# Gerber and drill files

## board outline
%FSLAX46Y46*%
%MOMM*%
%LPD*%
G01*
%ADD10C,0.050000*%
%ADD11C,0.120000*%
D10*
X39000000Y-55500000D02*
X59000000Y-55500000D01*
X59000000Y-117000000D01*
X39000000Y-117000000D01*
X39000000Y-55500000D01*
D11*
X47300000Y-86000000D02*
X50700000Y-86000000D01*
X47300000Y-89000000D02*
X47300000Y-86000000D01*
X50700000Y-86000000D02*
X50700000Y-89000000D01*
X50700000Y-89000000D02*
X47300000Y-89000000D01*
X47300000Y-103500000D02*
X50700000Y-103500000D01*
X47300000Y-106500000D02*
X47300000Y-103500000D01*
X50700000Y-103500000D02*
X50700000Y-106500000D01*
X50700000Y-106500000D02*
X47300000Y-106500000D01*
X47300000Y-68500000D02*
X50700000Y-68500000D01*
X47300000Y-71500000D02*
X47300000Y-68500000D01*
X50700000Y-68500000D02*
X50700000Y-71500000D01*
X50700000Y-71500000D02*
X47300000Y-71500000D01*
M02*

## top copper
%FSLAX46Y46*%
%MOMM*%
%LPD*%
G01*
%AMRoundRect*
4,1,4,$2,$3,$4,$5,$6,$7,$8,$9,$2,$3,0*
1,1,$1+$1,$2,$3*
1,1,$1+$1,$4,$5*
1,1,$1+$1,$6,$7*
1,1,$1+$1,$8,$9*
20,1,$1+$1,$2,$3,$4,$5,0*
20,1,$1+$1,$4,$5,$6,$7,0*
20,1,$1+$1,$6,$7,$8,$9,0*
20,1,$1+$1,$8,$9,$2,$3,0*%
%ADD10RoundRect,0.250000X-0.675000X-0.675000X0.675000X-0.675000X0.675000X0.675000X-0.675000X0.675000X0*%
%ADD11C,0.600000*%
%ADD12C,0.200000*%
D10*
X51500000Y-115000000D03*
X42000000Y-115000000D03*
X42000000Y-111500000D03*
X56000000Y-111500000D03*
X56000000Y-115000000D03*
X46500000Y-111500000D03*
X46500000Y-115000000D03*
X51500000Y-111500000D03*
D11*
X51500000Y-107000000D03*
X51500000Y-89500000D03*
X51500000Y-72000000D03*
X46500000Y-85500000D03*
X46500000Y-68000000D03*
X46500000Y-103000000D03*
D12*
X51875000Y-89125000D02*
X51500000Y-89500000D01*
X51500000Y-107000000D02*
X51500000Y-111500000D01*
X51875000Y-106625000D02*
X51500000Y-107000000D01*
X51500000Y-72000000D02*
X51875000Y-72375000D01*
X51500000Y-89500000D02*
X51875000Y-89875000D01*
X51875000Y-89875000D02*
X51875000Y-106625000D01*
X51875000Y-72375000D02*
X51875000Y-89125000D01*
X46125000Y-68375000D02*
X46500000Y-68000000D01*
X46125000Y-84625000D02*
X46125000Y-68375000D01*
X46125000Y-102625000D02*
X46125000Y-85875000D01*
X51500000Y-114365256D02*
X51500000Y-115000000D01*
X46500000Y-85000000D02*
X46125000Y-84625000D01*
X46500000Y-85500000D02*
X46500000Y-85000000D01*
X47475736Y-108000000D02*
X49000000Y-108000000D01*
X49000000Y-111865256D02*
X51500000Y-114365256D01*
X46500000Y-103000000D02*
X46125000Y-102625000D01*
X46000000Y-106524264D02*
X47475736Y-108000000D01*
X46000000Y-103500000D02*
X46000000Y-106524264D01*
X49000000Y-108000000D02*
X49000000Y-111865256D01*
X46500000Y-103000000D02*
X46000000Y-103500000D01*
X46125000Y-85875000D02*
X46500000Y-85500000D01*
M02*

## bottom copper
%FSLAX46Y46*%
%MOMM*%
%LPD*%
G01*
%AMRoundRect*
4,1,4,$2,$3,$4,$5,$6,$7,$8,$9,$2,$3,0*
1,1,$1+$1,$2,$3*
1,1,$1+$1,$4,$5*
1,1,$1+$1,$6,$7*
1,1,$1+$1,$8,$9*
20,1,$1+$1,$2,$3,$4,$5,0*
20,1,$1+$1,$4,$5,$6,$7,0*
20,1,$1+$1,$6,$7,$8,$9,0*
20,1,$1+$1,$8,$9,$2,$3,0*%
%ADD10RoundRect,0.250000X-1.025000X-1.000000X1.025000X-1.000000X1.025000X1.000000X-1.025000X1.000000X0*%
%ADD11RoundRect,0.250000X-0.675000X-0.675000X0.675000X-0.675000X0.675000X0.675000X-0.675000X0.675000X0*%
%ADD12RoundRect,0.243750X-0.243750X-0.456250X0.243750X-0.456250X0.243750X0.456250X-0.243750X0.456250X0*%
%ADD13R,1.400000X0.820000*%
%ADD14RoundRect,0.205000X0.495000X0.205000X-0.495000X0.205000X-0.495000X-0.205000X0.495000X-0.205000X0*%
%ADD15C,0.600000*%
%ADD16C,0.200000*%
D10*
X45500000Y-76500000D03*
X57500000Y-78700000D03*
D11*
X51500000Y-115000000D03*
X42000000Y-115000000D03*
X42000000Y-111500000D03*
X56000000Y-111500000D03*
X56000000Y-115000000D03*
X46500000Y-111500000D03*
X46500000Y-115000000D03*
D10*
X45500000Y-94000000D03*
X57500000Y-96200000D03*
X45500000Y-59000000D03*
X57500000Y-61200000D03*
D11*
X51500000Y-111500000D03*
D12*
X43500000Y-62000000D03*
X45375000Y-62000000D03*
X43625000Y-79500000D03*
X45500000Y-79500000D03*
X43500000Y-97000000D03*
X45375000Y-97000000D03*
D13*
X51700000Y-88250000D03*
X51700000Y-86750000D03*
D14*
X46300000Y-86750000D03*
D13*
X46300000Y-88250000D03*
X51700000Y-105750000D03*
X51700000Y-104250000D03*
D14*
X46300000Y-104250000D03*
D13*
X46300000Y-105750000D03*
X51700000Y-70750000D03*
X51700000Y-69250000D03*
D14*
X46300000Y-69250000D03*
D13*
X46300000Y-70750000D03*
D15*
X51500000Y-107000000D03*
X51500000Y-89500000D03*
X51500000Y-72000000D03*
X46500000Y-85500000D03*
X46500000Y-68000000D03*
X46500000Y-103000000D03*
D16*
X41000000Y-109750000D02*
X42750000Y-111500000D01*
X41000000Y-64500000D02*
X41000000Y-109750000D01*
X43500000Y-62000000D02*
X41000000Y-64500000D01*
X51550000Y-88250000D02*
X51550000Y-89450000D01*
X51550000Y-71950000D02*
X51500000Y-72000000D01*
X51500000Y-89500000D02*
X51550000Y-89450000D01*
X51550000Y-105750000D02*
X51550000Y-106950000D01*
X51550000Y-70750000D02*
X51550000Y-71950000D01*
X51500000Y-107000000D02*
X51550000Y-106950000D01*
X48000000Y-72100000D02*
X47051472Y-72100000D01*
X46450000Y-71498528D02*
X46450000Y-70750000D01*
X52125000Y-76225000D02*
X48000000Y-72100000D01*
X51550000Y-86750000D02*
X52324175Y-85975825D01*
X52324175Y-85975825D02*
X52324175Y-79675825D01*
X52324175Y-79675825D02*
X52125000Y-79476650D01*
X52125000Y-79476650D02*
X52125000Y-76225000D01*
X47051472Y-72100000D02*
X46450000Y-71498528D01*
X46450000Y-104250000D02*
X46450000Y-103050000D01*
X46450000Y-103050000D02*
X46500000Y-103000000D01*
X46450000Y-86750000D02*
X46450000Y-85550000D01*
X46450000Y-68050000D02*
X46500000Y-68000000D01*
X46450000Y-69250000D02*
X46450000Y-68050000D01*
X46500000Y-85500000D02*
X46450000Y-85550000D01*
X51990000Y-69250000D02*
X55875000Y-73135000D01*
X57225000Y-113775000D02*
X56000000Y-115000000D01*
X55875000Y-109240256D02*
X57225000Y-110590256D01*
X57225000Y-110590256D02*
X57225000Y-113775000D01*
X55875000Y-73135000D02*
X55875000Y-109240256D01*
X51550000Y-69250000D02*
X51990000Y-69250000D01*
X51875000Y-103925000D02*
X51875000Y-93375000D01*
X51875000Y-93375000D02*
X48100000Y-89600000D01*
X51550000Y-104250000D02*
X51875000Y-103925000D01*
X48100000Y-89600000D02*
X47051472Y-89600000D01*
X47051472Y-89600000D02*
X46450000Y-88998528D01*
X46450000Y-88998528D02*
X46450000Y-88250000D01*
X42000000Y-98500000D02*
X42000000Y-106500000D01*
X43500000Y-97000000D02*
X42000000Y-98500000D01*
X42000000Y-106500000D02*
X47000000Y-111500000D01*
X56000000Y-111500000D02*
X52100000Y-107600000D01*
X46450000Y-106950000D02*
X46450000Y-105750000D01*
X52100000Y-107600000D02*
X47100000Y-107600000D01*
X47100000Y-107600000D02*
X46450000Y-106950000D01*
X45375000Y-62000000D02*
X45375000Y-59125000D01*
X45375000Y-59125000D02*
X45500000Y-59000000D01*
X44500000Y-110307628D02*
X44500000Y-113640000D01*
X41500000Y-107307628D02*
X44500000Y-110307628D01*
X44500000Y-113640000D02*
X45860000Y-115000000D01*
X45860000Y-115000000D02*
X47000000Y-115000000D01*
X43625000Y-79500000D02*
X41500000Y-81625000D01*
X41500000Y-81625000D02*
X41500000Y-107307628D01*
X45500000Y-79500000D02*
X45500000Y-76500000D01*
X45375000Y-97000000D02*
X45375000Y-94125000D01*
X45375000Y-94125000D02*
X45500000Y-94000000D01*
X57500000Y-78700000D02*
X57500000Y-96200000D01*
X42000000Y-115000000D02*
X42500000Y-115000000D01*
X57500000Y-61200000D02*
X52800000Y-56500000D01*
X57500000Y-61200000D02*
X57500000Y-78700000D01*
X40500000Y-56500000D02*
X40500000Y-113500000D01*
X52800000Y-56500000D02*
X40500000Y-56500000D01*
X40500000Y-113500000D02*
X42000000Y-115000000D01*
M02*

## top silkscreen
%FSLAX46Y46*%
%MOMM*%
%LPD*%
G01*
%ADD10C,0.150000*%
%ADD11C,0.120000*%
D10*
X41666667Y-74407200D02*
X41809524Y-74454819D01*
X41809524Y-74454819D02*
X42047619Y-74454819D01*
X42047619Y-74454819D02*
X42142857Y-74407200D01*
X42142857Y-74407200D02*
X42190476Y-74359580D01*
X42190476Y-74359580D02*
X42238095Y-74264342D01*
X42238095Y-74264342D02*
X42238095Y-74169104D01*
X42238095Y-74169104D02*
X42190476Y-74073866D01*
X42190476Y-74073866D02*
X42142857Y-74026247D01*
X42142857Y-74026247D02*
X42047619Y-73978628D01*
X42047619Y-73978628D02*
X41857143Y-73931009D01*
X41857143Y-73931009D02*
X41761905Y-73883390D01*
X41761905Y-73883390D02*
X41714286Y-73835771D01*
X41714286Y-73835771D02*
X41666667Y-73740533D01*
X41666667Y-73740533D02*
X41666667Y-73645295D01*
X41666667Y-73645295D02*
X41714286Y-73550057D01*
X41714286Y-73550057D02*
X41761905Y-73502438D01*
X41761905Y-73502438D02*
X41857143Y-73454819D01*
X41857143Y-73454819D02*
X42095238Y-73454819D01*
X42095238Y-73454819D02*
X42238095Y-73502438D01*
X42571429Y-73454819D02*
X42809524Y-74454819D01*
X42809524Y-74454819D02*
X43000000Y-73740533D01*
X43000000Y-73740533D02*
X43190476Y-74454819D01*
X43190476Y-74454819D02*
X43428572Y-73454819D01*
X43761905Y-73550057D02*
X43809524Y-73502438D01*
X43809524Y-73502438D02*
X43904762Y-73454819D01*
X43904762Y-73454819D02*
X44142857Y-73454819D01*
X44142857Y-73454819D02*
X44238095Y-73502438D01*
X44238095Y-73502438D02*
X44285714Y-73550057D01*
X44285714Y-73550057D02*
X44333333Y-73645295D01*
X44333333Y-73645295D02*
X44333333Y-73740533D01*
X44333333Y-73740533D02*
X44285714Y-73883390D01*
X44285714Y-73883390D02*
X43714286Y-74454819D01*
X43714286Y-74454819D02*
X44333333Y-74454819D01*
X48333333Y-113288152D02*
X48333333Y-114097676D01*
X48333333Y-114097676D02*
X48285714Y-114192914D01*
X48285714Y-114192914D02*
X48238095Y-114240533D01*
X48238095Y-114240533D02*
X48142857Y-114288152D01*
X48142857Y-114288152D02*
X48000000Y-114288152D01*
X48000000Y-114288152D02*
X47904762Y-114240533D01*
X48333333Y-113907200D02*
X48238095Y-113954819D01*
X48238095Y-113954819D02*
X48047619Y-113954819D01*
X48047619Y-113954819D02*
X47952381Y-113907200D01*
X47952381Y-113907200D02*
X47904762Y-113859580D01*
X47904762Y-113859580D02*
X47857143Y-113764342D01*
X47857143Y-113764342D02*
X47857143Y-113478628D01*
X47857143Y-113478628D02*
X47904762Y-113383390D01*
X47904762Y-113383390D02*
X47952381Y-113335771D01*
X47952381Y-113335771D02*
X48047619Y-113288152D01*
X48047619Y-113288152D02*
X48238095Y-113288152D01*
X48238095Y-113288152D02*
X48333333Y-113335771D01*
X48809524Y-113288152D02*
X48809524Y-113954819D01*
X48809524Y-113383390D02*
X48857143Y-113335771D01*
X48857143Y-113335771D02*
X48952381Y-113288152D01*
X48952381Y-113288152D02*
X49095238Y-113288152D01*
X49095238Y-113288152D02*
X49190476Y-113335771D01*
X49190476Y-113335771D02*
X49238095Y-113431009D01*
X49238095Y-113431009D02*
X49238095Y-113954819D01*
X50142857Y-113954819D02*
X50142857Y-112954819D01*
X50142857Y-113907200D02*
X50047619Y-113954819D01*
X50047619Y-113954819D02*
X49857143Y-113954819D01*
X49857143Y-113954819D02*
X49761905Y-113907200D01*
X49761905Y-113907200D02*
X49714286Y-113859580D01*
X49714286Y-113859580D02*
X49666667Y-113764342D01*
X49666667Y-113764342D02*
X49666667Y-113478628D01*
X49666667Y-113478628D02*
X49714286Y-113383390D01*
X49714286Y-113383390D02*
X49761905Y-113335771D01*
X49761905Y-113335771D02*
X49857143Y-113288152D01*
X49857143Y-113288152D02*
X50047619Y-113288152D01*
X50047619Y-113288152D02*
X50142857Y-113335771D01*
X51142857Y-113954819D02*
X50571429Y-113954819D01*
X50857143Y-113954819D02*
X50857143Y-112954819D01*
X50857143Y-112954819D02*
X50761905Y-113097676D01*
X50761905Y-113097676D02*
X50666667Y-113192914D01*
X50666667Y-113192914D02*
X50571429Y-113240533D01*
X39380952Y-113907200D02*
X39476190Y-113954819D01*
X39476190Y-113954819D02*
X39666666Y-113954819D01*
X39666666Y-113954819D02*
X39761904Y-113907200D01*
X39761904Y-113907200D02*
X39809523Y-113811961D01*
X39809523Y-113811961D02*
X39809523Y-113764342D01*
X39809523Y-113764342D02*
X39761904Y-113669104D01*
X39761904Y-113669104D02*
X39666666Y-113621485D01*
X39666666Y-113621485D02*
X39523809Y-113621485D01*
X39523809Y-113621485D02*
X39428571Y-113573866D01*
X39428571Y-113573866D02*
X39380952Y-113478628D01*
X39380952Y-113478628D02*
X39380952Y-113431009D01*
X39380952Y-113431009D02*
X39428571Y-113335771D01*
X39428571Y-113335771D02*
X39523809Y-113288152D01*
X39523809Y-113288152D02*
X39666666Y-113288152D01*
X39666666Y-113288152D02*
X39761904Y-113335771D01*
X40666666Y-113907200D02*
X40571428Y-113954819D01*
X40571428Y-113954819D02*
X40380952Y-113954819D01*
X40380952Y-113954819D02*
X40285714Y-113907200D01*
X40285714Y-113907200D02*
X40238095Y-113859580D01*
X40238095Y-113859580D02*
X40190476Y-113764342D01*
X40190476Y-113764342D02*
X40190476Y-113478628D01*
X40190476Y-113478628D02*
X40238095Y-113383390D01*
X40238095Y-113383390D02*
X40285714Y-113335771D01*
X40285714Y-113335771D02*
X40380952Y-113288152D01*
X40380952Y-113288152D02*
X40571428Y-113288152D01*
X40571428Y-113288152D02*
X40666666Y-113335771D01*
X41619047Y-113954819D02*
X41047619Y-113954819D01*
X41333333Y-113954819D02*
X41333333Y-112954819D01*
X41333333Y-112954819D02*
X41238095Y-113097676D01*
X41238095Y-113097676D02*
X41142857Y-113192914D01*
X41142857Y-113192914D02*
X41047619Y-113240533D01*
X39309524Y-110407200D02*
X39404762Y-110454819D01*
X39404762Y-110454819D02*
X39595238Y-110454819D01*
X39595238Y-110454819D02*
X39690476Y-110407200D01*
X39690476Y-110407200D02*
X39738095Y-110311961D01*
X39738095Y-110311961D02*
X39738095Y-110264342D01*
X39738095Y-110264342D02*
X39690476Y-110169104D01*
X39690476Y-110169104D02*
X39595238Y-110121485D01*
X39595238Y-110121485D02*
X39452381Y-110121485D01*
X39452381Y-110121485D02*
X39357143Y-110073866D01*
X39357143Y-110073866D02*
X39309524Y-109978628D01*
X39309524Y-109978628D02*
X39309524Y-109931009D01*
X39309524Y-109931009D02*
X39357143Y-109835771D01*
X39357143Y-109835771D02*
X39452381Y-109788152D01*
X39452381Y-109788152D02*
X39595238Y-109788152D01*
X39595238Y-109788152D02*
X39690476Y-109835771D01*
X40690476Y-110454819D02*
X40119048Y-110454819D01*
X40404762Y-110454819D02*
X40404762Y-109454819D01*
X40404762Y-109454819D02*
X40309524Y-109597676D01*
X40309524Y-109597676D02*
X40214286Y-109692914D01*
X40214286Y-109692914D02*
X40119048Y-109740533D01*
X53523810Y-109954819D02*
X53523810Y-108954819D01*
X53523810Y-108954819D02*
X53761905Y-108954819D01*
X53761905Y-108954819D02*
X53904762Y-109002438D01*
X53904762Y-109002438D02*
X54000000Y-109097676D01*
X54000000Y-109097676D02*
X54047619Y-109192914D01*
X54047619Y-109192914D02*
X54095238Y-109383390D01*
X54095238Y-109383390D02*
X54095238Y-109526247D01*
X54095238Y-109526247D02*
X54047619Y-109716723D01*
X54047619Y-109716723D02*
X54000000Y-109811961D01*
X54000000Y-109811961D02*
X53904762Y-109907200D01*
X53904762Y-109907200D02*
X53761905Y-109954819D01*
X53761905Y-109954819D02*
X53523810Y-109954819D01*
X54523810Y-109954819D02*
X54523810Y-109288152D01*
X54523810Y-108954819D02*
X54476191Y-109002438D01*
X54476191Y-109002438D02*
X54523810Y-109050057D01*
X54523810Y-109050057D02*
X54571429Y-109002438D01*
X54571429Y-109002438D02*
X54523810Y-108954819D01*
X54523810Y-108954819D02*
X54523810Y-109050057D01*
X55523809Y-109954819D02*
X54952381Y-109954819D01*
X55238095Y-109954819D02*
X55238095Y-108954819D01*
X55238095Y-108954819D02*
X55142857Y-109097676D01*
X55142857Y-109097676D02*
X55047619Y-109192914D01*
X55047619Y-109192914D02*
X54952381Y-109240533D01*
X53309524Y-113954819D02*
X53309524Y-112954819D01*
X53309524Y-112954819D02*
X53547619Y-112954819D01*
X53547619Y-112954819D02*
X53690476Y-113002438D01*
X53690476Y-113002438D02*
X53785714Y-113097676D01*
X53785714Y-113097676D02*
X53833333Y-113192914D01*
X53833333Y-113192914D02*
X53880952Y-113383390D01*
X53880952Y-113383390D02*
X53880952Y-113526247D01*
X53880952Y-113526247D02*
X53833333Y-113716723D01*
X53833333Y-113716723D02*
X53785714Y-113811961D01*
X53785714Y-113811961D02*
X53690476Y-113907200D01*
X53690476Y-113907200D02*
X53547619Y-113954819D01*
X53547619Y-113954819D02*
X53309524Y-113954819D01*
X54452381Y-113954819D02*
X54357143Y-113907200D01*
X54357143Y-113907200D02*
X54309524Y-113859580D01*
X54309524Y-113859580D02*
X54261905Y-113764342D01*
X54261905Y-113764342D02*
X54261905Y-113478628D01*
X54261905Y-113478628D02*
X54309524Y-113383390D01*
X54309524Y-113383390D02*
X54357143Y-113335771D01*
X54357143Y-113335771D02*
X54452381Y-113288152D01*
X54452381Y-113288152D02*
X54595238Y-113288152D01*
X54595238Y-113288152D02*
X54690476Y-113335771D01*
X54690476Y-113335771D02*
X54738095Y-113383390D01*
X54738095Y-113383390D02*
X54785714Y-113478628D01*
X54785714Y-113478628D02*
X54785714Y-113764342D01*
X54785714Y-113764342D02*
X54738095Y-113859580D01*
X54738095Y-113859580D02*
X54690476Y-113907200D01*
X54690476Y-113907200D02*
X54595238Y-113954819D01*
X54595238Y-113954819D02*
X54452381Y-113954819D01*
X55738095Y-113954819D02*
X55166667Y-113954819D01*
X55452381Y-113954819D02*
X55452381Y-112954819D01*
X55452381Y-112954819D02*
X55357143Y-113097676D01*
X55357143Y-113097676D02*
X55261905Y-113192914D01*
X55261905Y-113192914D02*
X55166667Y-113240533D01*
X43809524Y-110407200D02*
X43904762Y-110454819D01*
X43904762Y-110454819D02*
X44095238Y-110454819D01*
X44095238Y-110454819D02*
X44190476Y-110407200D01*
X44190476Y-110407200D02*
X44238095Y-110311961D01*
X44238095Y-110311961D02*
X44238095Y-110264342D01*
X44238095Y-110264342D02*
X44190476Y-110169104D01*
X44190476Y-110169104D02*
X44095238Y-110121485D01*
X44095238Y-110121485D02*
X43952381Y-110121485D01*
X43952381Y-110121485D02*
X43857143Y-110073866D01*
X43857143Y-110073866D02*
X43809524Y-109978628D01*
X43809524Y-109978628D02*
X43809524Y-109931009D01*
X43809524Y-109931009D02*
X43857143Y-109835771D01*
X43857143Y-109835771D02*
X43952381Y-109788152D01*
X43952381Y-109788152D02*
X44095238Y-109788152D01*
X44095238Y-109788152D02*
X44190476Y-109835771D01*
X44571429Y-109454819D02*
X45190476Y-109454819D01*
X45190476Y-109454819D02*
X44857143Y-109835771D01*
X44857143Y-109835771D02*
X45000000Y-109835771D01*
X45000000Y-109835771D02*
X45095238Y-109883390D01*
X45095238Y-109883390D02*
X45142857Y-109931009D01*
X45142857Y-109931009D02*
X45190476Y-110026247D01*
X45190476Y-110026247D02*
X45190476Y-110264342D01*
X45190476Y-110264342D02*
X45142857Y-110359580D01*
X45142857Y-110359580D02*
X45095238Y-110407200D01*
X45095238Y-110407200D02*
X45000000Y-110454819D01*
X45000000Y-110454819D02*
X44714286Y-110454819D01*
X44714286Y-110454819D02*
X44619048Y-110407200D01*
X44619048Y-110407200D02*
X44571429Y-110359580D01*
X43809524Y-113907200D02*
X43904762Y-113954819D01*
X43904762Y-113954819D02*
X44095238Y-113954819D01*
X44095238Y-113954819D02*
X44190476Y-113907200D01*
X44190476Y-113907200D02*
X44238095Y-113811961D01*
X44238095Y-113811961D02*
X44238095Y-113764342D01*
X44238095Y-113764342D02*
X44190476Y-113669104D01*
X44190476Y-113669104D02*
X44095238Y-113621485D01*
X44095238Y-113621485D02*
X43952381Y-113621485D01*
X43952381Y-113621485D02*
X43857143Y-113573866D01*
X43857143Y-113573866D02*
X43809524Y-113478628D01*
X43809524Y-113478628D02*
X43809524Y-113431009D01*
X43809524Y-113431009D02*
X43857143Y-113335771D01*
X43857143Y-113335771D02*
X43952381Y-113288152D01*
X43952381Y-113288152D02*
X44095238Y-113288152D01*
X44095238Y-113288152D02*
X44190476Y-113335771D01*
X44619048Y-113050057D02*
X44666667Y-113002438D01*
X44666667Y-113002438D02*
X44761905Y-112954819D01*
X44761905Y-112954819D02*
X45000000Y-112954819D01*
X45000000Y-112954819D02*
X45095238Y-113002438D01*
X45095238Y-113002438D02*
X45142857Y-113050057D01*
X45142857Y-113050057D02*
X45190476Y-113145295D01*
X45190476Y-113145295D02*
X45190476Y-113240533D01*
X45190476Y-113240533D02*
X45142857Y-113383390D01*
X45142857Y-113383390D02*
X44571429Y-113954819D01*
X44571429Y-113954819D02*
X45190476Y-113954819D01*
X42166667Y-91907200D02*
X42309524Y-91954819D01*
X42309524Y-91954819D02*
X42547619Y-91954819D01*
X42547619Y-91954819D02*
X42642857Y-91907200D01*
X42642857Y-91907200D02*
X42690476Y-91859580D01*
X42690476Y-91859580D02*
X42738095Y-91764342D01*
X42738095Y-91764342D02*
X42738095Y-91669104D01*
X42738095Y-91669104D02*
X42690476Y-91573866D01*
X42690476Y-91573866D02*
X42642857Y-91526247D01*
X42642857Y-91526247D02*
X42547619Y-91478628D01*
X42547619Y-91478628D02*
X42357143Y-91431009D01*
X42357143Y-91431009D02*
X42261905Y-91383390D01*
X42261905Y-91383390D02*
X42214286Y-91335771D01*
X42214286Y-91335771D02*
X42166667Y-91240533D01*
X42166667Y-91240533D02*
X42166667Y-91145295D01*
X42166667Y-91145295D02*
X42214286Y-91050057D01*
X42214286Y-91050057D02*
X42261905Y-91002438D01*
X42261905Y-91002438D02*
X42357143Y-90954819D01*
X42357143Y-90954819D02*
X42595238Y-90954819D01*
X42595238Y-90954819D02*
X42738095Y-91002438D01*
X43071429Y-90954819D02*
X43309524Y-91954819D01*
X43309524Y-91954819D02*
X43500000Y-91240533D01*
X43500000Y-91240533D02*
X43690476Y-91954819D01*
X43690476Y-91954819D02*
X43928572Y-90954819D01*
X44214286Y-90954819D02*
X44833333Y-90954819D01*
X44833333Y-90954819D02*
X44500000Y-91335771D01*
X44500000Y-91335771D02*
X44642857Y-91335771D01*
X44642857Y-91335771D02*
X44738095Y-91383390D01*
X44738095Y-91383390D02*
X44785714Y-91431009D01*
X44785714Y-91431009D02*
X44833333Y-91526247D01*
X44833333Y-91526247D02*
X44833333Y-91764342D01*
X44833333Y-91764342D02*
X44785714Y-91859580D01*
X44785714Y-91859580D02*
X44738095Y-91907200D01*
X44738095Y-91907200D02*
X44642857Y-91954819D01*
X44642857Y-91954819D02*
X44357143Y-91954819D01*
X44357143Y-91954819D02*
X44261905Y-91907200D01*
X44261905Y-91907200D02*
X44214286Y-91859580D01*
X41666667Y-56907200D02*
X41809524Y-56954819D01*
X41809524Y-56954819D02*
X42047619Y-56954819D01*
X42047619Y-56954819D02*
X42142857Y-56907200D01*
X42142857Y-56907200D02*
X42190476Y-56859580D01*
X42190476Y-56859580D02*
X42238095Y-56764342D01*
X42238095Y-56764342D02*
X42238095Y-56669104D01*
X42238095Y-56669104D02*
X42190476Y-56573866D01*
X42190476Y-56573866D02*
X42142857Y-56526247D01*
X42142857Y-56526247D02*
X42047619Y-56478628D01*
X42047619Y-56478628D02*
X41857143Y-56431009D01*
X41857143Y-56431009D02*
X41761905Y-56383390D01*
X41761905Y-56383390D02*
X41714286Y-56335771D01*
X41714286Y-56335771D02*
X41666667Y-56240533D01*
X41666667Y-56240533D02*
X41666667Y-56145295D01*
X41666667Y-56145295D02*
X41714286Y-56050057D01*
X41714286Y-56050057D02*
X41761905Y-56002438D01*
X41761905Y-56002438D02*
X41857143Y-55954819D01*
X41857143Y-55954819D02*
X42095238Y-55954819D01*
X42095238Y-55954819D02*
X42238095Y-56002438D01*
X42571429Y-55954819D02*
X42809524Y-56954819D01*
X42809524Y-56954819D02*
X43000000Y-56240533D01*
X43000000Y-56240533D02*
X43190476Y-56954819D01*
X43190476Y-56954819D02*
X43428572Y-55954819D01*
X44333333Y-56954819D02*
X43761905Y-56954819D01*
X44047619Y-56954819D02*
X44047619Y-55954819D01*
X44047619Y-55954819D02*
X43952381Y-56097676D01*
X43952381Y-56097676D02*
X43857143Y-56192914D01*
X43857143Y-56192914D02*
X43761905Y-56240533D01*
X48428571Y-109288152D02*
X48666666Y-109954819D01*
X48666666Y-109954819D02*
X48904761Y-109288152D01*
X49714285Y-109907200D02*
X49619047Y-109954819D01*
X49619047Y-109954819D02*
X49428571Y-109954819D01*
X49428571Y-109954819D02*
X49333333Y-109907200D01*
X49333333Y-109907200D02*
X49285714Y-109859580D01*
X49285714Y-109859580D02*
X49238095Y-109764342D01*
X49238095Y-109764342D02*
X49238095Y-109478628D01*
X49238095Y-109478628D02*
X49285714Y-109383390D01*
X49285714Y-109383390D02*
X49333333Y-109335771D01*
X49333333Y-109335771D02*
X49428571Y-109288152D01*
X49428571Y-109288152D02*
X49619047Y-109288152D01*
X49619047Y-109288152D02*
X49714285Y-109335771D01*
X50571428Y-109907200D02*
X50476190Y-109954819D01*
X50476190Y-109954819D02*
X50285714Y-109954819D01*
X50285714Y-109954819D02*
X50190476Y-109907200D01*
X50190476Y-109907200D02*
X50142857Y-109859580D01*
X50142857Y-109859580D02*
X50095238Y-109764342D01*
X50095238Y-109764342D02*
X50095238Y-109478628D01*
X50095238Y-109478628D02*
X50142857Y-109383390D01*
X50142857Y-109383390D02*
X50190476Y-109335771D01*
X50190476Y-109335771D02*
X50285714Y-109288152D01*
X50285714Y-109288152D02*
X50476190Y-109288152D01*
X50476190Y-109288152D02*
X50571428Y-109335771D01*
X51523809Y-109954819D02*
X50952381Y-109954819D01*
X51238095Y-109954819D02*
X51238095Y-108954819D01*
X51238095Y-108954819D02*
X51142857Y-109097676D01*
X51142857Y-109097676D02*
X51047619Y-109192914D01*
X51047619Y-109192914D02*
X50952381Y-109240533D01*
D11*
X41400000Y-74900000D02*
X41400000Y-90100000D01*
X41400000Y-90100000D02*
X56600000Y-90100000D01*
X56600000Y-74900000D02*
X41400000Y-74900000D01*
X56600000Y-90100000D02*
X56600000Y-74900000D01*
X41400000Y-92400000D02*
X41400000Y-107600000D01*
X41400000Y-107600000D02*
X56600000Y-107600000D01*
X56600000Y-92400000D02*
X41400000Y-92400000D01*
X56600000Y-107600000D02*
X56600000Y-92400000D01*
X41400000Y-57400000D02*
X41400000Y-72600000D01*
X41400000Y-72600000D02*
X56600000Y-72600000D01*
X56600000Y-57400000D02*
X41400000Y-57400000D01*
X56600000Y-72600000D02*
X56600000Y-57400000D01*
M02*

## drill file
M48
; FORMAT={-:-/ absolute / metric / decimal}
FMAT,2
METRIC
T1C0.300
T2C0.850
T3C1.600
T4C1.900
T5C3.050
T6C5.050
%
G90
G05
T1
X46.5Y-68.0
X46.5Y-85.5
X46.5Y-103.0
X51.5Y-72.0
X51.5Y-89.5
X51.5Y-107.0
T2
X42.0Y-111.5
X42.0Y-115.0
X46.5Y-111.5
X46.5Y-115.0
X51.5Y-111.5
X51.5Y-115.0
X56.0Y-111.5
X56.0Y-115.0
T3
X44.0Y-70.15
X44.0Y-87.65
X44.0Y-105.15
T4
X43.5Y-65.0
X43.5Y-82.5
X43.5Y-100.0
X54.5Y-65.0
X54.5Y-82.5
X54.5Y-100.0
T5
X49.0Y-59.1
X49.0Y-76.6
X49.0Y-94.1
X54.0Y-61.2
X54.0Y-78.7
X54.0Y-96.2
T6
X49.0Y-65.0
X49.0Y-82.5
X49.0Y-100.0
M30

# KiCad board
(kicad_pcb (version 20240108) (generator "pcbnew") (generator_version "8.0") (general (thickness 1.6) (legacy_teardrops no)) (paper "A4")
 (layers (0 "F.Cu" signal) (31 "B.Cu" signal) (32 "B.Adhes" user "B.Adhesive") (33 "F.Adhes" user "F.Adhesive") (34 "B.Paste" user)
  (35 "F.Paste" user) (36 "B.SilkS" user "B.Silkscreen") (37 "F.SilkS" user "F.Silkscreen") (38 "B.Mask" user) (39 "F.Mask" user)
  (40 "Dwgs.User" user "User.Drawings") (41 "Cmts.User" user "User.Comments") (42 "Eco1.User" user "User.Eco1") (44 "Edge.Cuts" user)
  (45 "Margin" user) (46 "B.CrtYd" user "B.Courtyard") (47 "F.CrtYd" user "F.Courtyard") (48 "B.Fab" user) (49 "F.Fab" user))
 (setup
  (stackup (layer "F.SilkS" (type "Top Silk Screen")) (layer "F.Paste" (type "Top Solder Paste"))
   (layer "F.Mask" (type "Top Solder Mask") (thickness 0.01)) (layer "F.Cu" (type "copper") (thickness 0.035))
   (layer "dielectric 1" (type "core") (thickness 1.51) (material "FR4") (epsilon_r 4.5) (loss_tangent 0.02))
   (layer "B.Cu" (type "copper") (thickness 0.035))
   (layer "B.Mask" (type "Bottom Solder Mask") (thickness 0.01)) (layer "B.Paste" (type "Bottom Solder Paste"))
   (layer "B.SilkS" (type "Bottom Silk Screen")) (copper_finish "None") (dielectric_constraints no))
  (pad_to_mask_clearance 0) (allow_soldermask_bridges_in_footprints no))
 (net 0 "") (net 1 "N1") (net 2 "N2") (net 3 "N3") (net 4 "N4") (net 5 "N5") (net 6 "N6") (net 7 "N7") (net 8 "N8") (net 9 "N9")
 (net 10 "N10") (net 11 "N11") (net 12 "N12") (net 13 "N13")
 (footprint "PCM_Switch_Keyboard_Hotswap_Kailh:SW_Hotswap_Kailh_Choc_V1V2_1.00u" (layer "F.Cu") (at 49 82.5)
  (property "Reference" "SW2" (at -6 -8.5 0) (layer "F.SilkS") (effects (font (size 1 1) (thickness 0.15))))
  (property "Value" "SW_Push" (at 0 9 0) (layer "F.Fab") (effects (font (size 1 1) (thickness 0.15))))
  (fp_line (start -7.6 -7.6) (end -7.6 7.6) (stroke (width 0.12) (type solid)) (layer "F.SilkS"))
  (fp_line (start -7.6 7.6) (end 7.6 7.6) (stroke (width 0.12) (type solid)) (layer "F.SilkS"))
  (fp_line (start 7.6 -7.6) (end -7.6 -7.6) (stroke (width 0.12) (type solid)) (layer "F.SilkS"))
  (fp_line (start 7.6 7.6) (end 7.6 -7.6) (stroke (width 0.12) (type solid)) (layer "F.SilkS"))
  (pad "" np_thru_hole circle (at -5.5 0) (size 1.9 1.9) (drill 1.9) (layers "*.Cu" "*.Mask"))
  (pad "" np_thru_hole circle (at -5 5.15) (size 1.6 1.6) (drill 1.6) (layers "*.Cu" "*.Mask"))
  (pad "" np_thru_hole circle (at 0 -5.9) (size 3.05 3.05) (drill 3.05) (layers "*.Cu" "*.Mask"))
  (pad "" np_thru_hole circle (at 0 0) (size 5.05 5.05) (drill 5.05) (layers "*.Cu" "*.Mask"))
  (pad "" np_thru_hole circle (at 5 -3.8) (size 3.05 3.05) (drill 3.05) (layers "*.Cu" "*.Mask"))
  (pad "" np_thru_hole circle (at 5.5 0) (size 1.9 1.9) (drill 1.9) (layers "*.Cu" "*.Mask"))
  (pad "1" smd roundrect (at -3.5 -6) (size 2.55 2.5) (layers "B.Cu" "B.Paste" "B.Mask") (roundrect_rratio 0.1) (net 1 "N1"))
  (pad "2" smd roundrect (at 8.5 -3.8) (size 2.55 2.5) (layers "B.Cu" "B.Paste" "B.Mask") (roundrect_rratio 0.1) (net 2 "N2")))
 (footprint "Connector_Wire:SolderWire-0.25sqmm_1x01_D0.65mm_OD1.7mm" (layer "F.Cu") (at 51.5 115)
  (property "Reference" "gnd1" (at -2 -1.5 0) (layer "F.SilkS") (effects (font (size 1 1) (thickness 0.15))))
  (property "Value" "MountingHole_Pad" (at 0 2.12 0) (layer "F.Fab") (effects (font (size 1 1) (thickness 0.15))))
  (pad "1" thru_hole roundrect (at 0 0) (size 1.85 1.85) (drill 0.85) (layers "*.Cu" "*.Mask") (remove_unused_layers no)
   (roundrect_rratio 0.135135) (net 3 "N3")))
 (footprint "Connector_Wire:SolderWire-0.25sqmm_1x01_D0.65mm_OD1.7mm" (layer "F.Cu") (at 42 115)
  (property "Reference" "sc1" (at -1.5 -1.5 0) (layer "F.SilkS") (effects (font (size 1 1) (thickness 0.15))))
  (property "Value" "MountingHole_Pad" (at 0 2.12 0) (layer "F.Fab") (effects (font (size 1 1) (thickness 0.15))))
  (pad "1" thru_hole roundrect (at 0 0) (size 1.85 1.85) (drill 0.85) (layers "*.Cu" "*.Mask") (remove_unused_layers no)
   (roundrect_rratio 0.135135) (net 2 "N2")))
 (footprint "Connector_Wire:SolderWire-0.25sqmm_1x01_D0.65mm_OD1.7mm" (layer "F.Cu") (at 42 111.5)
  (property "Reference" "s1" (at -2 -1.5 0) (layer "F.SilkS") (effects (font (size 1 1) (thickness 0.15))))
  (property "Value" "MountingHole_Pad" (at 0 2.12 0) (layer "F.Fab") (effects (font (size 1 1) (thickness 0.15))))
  (pad "1" thru_hole roundrect (at 0 0) (size 1.85 1.85) (drill 0.85) (layers "*.Cu" "*.Mask") (remove_unused_layers no)
   (roundrect_rratio 0.135135) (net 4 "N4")))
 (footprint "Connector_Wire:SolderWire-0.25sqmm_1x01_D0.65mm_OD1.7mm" (layer "F.Cu") (at 56 111.5)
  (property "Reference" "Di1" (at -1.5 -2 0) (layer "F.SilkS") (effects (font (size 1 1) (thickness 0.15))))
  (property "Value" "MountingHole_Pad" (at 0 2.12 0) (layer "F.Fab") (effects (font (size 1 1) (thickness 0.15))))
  (pad "1" thru_hole roundrect (at 0 0) (size 1.85 1.85) (drill 0.85) (layers "*.Cu" "*.Mask") (remove_unused_layers no)
   (roundrect_rratio 0.135135) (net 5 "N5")))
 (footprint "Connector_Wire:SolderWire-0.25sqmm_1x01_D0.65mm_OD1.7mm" (layer "F.Cu") (at 56 115)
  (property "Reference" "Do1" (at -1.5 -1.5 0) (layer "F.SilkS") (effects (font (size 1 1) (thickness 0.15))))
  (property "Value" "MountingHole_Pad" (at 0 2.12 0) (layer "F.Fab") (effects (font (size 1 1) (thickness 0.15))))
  (pad "1" thru_hole roundrect (at 0 0) (size 1.85 1.85) (drill 0.85) (layers "*.Cu" "*.Mask") (remove_unused_layers no)
   (roundrect_rratio 0.135135) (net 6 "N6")))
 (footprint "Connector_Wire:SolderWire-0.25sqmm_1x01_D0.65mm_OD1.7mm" (layer "F.Cu") (at 46.5 111.5)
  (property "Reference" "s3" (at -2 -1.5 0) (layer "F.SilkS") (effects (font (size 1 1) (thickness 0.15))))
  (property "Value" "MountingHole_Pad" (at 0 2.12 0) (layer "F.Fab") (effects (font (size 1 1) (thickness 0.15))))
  (pad "1" thru_hole roundrect (at 0 0) (size 1.85 1.85) (drill 0.85) (layers "*.Cu" "*.Mask") (remove_unused_layers no)
   (roundrect_rratio 0.135135) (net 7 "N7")))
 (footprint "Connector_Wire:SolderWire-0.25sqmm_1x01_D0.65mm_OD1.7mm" (layer "F.Cu") (at 46.5 115)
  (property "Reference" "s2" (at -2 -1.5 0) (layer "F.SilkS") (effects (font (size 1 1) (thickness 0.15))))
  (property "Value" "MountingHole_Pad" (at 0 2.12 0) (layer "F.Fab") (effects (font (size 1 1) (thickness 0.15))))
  (pad "1" thru_hole roundrect (at 0 0) (size 1.85 1.85) (drill 0.85) (layers "*.Cu" "*.Mask") (remove_unused_layers no)
   (roundrect_rratio 0.135135) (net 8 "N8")))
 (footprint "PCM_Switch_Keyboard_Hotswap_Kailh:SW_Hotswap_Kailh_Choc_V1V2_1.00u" (layer "F.Cu") (at 49 100)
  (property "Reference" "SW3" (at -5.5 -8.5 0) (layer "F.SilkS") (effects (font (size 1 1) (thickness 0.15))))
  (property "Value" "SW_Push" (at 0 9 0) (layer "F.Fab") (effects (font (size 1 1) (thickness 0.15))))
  (fp_line (start -7.6 -7.6) (end -7.6 7.6) (stroke (width 0.12) (type solid)) (layer "F.SilkS"))
  (fp_line (start -7.6 7.6) (end 7.6 7.6) (stroke (width 0.12) (type solid)) (layer "F.SilkS"))
  (fp_line (start 7.6 -7.6) (end -7.6 -7.6) (stroke (width 0.12) (type solid)) (layer "F.SilkS"))
  (fp_line (start 7.6 7.6) (end 7.6 -7.6) (stroke (width 0.12) (type solid)) (layer "F.SilkS"))
  (pad "" np_thru_hole circle (at -5.5 0) (size 1.9 1.9) (drill 1.9) (layers "*.Cu" "*.Mask"))
  (pad "" np_thru_hole circle (at -5 5.15) (size 1.6 1.6) (drill 1.6) (layers "*.Cu" "*.Mask"))
  (pad "" np_thru_hole circle (at 0 -5.9) (size 3.05 3.05) (drill 3.05) (layers "*.Cu" "*.Mask"))
  (pad "" np_thru_hole circle (at 0 0) (size 5.05 5.05) (drill 5.05) (layers "*.Cu" "*.Mask"))
  (pad "" np_thru_hole circle (at 5 -3.8) (size 3.05 3.05) (drill 3.05) (layers "*.Cu" "*.Mask"))
  (pad "" np_thru_hole circle (at 5.5 0) (size 1.9 1.9) (drill 1.9) (layers "*.Cu" "*.Mask"))
  (pad "1" smd roundrect (at -3.5 -6) (size 2.55 2.5) (layers "B.Cu" "B.Paste" "B.Mask") (roundrect_rratio 0.1) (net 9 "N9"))
  (pad "2" smd roundrect (at 8.5 -3.8) (size 2.55 2.5) (layers "B.Cu" "B.Paste" "B.Mask") (roundrect_rratio 0.1) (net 2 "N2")))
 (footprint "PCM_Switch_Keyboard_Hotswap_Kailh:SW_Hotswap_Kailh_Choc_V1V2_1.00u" (layer "F.Cu") (at 49 65)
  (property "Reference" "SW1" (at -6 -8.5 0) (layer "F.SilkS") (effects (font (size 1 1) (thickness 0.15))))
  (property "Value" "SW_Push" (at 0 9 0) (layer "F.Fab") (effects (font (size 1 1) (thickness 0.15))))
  (fp_line (start -7.6 -7.6) (end -7.6 7.6) (stroke (width 0.12) (type solid)) (layer "F.SilkS"))
  (fp_line (start -7.6 7.6) (end 7.6 7.6) (stroke (width 0.12) (type solid)) (layer "F.SilkS"))
  (fp_line (start 7.6 -7.6) (end -7.6 -7.6) (stroke (width 0.12) (type solid)) (layer "F.SilkS"))
  (fp_line (start 7.6 7.6) (end 7.6 -7.6) (stroke (width 0.12) (type solid)) (layer "F.SilkS"))
  (pad "" np_thru_hole circle (at -5.5 0) (size 1.9 1.9) (drill 1.9) (layers "*.Cu" "*.Mask"))
  (pad "" np_thru_hole circle (at -5 5.15) (size 1.6 1.6) (drill 1.6) (layers "*.Cu" "*.Mask"))
  (pad "" np_thru_hole circle (at 0 -5.9) (size 3.05 3.05) (drill 3.05) (layers "*.Cu" "*.Mask"))
  (pad "" np_thru_hole circle (at 0 0) (size 5.05 5.05) (drill 5.05) (layers "*.Cu" "*.Mask"))
  (pad "" np_thru_hole circle (at 5 -3.8) (size 3.05 3.05) (drill 3.05) (layers "*.Cu" "*.Mask"))
  (pad "" np_thru_hole circle (at 5.5 0) (size 1.9 1.9) (drill 1.9) (layers "*.Cu" "*.Mask"))
  (pad "1" smd roundrect (at -3.5 -6) (size 2.55 2.5) (layers "B.Cu" "B.Paste" "B.Mask") (roundrect_rratio 0.1) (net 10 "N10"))
  (pad "2" smd roundrect (at 8.5 -3.8) (size 2.55 2.5) (layers "B.Cu" "B.Paste" "B.Mask") (roundrect_rratio 0.1) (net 2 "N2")))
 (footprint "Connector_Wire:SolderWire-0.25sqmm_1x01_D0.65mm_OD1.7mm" (layer "F.Cu") (at 51.5 111.5)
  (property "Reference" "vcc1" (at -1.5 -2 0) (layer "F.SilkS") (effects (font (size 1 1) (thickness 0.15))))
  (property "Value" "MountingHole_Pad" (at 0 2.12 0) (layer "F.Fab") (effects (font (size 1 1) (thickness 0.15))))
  (pad "1" thru_hole roundrect (at 0 0) (size 1.85 1.85) (drill 0.85) (layers "*.Cu" "*.Mask") (remove_unused_layers no)
   (roundrect_rratio 0.135135) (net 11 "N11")))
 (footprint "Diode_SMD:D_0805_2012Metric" (layer "B.Cu") (at 44.4375 62)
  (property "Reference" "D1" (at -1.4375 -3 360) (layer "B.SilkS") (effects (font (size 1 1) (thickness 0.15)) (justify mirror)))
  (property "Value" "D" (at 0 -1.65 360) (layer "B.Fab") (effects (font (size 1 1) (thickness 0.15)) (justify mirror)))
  (pad "1" smd roundrect (at -0.9375 0) (size 0.975 1.4) (layers "B.Cu" "B.Paste" "B.Mask") (roundrect_rratio 0.25) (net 4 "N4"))
  (pad "2" smd roundrect (at 0.9375 0) (size 0.975 1.4) (layers "B.Cu" "B.Paste" "B.Mask") (roundrect_rratio 0.25) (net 10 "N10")))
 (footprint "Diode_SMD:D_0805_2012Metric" (layer "B.Cu") (at 44.5625 79.5)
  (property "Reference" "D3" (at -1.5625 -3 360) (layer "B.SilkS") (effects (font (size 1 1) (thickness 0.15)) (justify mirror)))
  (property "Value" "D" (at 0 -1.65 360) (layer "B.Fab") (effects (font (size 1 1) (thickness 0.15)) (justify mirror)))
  (pad "1" smd roundrect (at -0.9375 0) (size 0.975 1.4) (layers "B.Cu" "B.Paste" "B.Mask") (roundrect_rratio 0.25) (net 8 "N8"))
  (pad "2" smd roundrect (at 0.9375 0) (size 0.975 1.4) (layers "B.Cu" "B.Paste" "B.Mask") (roundrect_rratio 0.25) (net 1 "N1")))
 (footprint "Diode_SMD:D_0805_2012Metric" (layer "B.Cu") (at 44.4375 97)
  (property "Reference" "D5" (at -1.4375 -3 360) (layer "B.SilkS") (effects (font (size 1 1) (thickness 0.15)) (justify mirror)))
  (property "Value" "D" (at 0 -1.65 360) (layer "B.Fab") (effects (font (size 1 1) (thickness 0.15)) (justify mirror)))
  (pad "1" smd roundrect (at -0.9375 0) (size 0.975 1.4) (layers "B.Cu" "B.Paste" "B.Mask") (roundrect_rratio 0.25) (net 7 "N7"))
  (pad "2" smd roundrect (at 0.9375 0) (size 0.975 1.4) (layers "B.Cu" "B.Paste" "B.Mask") (roundrect_rratio 0.25) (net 9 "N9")))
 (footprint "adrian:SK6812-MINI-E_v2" (layer "B.Cu") (at 49 87.5 180)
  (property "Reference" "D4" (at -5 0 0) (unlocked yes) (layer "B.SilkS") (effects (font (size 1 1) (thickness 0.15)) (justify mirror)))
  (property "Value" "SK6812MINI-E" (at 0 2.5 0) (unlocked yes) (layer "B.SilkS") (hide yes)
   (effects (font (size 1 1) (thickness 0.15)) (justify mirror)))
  (fp_line (start 1.7 1.5) (end -1.7 1.5) (stroke (width 0.12) (type solid)) (layer "Edge.Cuts"))
  (fp_line (start 1.7 -1.5) (end 1.7 1.5) (stroke (width 0.12) (type solid)) (layer "Edge.Cuts"))
  (fp_line (start -1.7 1.5) (end -1.7 -1.5) (stroke (width 0.12) (type solid)) (layer "Edge.Cuts"))
  (fp_line (start -1.7 -1.5) (end 1.7 -1.5) (stroke (width 0.12) (type solid)) (layer "Edge.Cuts"))
  (pad "1" smd rect (at -2.7 -0.75 180) (size 1.4 0.82) (layers "B.Cu" "B.Paste" "B.Mask") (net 11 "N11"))
  (pad "2" smd rect (at -2.7 0.75 180) (size 1.4 0.82) (layers "B.Cu" "B.Paste" "B.Mask") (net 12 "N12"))
  (pad "3" smd roundrect (at 2.7 0.75 180) (size 1.4 0.82) (layers "B.Cu" "B.Paste" "B.Mask") (roundrect_rratio 0.25) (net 3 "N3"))
  (pad "4" smd rect (at 2.7 -0.75 180) (size 1.4 0.82) (layers "B.Cu" "B.Paste" "B.Mask") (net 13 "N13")))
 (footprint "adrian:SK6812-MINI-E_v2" (layer "B.Cu") (at 49 105 180)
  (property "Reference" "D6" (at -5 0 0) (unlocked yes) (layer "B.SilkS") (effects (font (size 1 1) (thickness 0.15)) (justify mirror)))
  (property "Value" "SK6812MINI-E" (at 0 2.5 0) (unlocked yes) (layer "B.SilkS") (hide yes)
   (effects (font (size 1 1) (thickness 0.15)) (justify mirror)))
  (fp_line (start 1.7 1.5) (end -1.7 1.5) (stroke (width 0.12) (type solid)) (layer "Edge.Cuts"))
  (fp_line (start 1.7 -1.5) (end 1.7 1.5) (stroke (width 0.12) (type solid)) (layer "Edge.Cuts"))
  (fp_line (start -1.7 1.5) (end -1.7 -1.5) (stroke (width 0.12) (type solid)) (layer "Edge.Cuts"))
  (fp_line (start -1.7 -1.5) (end 1.7 -1.5) (stroke (width 0.12) (type solid)) (layer "Edge.Cuts"))
  (pad "1" smd rect (at -2.7 -0.75 180) (size 1.4 0.82) (layers "B.Cu" "B.Paste" "B.Mask") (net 11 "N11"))
  (pad "2" smd rect (at -2.7 0.75 180) (size 1.4 0.82) (layers "B.Cu" "B.Paste" "B.Mask") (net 13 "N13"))
  (pad "3" smd roundrect (at 2.7 0.75 180) (size 1.4 0.82) (layers "B.Cu" "B.Paste" "B.Mask") (roundrect_rratio 0.25) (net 3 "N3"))
  (pad "4" smd rect (at 2.7 -0.75 180) (size 1.4 0.82) (layers "B.Cu" "B.Paste" "B.Mask") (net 5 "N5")))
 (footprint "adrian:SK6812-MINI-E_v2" (layer "B.Cu") (at 49 70 180)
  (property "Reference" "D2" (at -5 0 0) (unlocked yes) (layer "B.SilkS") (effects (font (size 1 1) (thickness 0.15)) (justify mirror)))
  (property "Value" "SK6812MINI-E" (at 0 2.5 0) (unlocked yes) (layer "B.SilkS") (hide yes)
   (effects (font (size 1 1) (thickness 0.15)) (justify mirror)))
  (fp_line (start 1.7 1.5) (end -1.7 1.5) (stroke (width 0.12) (type solid)) (layer "Edge.Cuts"))
  (fp_line (start 1.7 -1.5) (end 1.7 1.5) (stroke (width 0.12) (type solid)) (layer "Edge.Cuts"))
  (fp_line (start -1.7 1.5) (end -1.7 -1.5) (stroke (width 0.12) (type solid)) (layer "Edge.Cuts"))
  (fp_line (start -1.7 -1.5) (end 1.7 -1.5) (stroke (width 0.12) (type solid)) (layer "Edge.Cuts"))
  (pad "1" smd rect (at -2.7 -0.75 180) (size 1.4 0.82) (layers "B.Cu" "B.Paste" "B.Mask") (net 11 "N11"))
  (pad "2" smd rect (at -2.7 0.75 180) (size 1.4 0.82) (layers "B.Cu" "B.Paste" "B.Mask") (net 6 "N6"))
  (pad "3" smd roundrect (at 2.7 0.75 180) (size 1.4 0.82) (layers "B.Cu" "B.Paste" "B.Mask") (roundrect_rratio 0.25) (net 3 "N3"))
  (pad "4" smd rect (at 2.7 -0.75 180) (size 1.4 0.82) (layers "B.Cu" "B.Paste" "B.Mask") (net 12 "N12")))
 (gr_rect (start 39 55.5) (end 59 117) (stroke (width 0.05) (type default)) (fill none) (layer "Edge.Cuts"))
 (segment (start 41 109.75) (end 42.75 111.5) (width 0.2) (layer "B.Cu") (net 4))
 (segment (start 41 64.5) (end 41 109.75) (width 0.2) (layer "B.Cu") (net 4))
 (segment (start 43.5 62) (end 41 64.5) (width 0.2) (layer "B.Cu") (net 4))
 (segment (start 51.875 89.125) (end 51.5 89.5) (width 0.2) (layer "F.Cu") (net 11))
 (segment (start 51.5 107) (end 51.5 111.5) (width 0.2) (layer "F.Cu") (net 11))
 (segment (start 51.875 106.625) (end 51.5 107) (width 0.2) (layer "F.Cu") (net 11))
 (segment (start 51.5 72) (end 51.875 72.375) (width 0.2) (layer "F.Cu") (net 11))
 (segment (start 51.5 89.5) (end 51.875 89.875) (width 0.2) (layer "F.Cu") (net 11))
 (segment (start 51.875 89.875) (end 51.875 106.625) (width 0.2) (layer "F.Cu") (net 11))
 (segment (start 51.875 72.375) (end 51.875 89.125) (width 0.2) (layer "F.Cu") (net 11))
 (via (at 51.5 107) (size 0.6) (drill 0.3) (layers "F.Cu" "B.Cu") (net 11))
 (via (at 51.5 89.5) (size 0.6) (drill 0.3) (layers "F.Cu" "B.Cu") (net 11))
 (via (at 51.5 72) (size 0.6) (drill 0.3) (layers "F.Cu" "B.Cu") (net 11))
 (segment (start 51.55 88.25) (end 51.55 89.45) (width 0.2) (layer "B.Cu") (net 11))
 (segment (start 51.55 71.95) (end 51.5 72) (width 0.2) (layer "B.Cu") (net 11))
 (segment (start 51.5 89.5) (end 51.55 89.45) (width 0.2) (layer "B.Cu") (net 11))
 (segment (start 51.55 105.75) (end 51.55 106.95) (width 0.2) (layer "B.Cu") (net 11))
 (segment (start 51.55 70.75) (end 51.55 71.95) (width 0.2) (layer "B.Cu") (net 11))
 (segment (start 51.5 107) (end 51.55 106.95) (width 0.2) (layer "B.Cu") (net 11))
 (segment (start 48 72.1) (end 47.051472 72.1) (width 0.2) (layer "B.Cu") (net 12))
 (segment (start 46.45 71.498528) (end 46.45 70.75) (width 0.2) (layer "B.Cu") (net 12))
 (segment (start 52.125 76.225) (end 48 72.1) (width 0.2) (layer "B.Cu") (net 12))
 (segment (start 51.55 86.75) (end 52.324175 85.975825) (width 0.2) (layer "B.Cu") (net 12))
 (segment (start 52.324175 85.975825) (end 52.324175 79.675825) (width 0.2) (layer "B.Cu") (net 12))
 (segment (start 52.324175 79.675825) (end 52.125 79.47665) (width 0.2) (layer "B.Cu") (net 12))
 (segment (start 52.125 79.47665) (end 52.125 76.225) (width 0.2) (layer "B.Cu") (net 12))
 (segment (start 47.051472 72.1) (end 46.45 71.498528) (width 0.2) (layer "B.Cu") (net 12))
 (segment (start 46.125 68.375) (end 46.5 68) (width 0.2) (layer "F.Cu") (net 3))
 (segment (start 46.125 84.625) (end 46.125 68.375) (width 0.2) (layer "F.Cu") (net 3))
 (segment (start 46.125 102.625) (end 46.125 85.875) (width 0.2) (layer "F.Cu") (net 3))
 (segment (start 51.5 114.365256) (end 51.5 115) (width 0.2) (layer "F.Cu") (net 3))
 (segment (start 46.5 85) (end 46.125 84.625) (width 0.2) (layer "F.Cu") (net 3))
 (segment (start 46.5 85.5) (end 46.5 85) (width 0.2) (layer "F.Cu") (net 3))
 (segment (start 47.475736 108) (end 49 108) (width 0.2) (layer "F.Cu") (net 3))
 (segment (start 49 111.865256) (end 51.5 114.365256) (width 0.2) (layer "F.Cu") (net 3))
 (segment (start 46.5 103) (end 46.125 102.625) (width 0.2) (layer "F.Cu") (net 3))
 (segment (start 46 106.524264) (end 47.475736 108) (width 0.2) (layer "F.Cu") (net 3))
 (segment (start 46 103.5) (end 46 106.524264) (width 0.2) (layer "F.Cu") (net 3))
 (segment (start 49 108) (end 49 111.865256) (width 0.2) (layer "F.Cu") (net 3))
 (segment (start 46.5 103) (end 46 103.5) (width 0.2) (layer "F.Cu") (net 3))
 (segment (start 46.125 85.875) (end 46.5 85.5) (width 0.2) (layer "F.Cu") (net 3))
 (via (at 46.5 85.5) (size 0.6) (drill 0.3) (layers "F.Cu" "B.Cu") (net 3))
 (via (at 46.5 68) (size 0.6) (drill 0.3) (layers "F.Cu" "B.Cu") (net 3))
 (via (at 46.5 103) (size 0.6) (drill 0.3) (layers "F.Cu" "B.Cu") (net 3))
 (segment (start 46.45 104.25) (end 46.45 103.05) (width 0.2) (layer "B.Cu") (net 3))
 (segment (start 46.45 103.05) (end 46.5 103) (width 0.2) (layer "B.Cu") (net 3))
 (segment (start 46.45 86.75) (end 46.45 85.55) (width 0.2) (layer "B.Cu") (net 3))
 (segment (start 46.45 68.05) (end 46.5 68) (width 0.2) (layer "B.Cu") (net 3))
 (segment (start 46.45 69.25) (end 46.45 68.05) (width 0.2) (layer "B.Cu") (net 3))
 (segment (start 46.5 85.5) (end 46.45 85.55) (width 0.2) (layer "B.Cu") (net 3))
 (segment (start 51.99 69.25) (end 55.875 73.135) (width 0.2) (layer "B.Cu") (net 6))
 (segment (start 57.225 113.775) (end 56 115) (width 0.2) (layer "B.Cu") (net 6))
 (segment (start 55.875 109.240256) (end 57.225 110.590256) (width 0.2) (layer "B.Cu") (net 6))
 (segment (start 57.225 110.590256) (end 57.225 113.775) (width 0.2) (layer "B.Cu") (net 6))
 (segment (start 55.875 73.135) (end 55.875 109.240256) (width 0.2) (layer "B.Cu") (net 6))
 (segment (start 51.55 69.25) (end 51.99 69.25) (width 0.2) (layer "B.Cu") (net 6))
 (segment (start 51.875 103.925) (end 51.875 93.375) (width 0.2) (layer "B.Cu") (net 13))
 (segment (start 51.875 93.375) (end 48.1 89.6) (width 0.2) (layer "B.Cu") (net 13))
 (segment (start 51.55 104.25) (end 51.875 103.925) (width 0.2) (layer "B.Cu") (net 13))
 (segment (start 48.1 89.6) (end 47.051472 89.6) (width 0.2) (layer "B.Cu") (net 13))
 (segment (start 47.051472 89.6) (end 46.45 88.998528) (width 0.2) (layer "B.Cu") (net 13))
 (segment (start 46.45 88.998528) (end 46.45 88.25) (width 0.2) (layer "B.Cu") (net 13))
 (segment (start 42 98.5) (end 42 106.5) (width 0.2) (layer "B.Cu") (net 7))
 (segment (start 43.5 97) (end 42 98.5) (width 0.2) (layer "B.Cu") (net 7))
 (segment (start 42 106.5) (end 47 111.5) (width 0.2) (layer "B.Cu") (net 7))
 (segment (start 56 111.5) (end 52.1 107.6) (width 0.2) (layer "B.Cu") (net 5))
 (segment (start 46.45 106.95) (end 46.45 105.75) (width 0.2) (layer "B.Cu") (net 5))
 (segment (start 52.1 107.6) (end 47.1 107.6) (width 0.2) (layer "B.Cu") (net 5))
 (segment (start 47.1 107.6) (end 46.45 106.95) (width 0.2) (layer "B.Cu") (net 5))
 (segment (start 45.375 62) (end 45.375 59.125) (width 0.2) (layer "B.Cu") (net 10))
 (segment (start 45.375 59.125) (end 45.5 59) (width 0.2) (layer "B.Cu") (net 10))
 (segment (start 44.5 110.307628) (end 44.5 113.64) (width 0.2) (layer "B.Cu") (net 8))
 (segment (start 41.5 107.307628) (end 44.5 110.307628) (width 0.2) (layer "B.Cu") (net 8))
 (segment (start 44.5 113.64) (end 45.86 115) (width 0.2) (layer "B.Cu") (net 8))
 (segment (start 45.86 115) (end 47 115) (width 0.2) (layer "B.Cu") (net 8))
 (segment (start 43.625 79.5) (end 41.5 81.625) (width 0.2) (layer "B.Cu") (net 8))
 (segment (start 41.5 81.625) (end 41.5 107.307628) (width 0.2) (layer "B.Cu") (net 8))
 (segment (start 45.5 79.5) (end 45.5 76.5) (width 0.2) (layer "B.Cu") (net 1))
 (segment (start 45.375 97) (end 45.375 94.125) (width 0.2) (layer "B.Cu") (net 9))
 (segment (start 45.375 94.125) (end 45.5 94) (width 0.2) (layer "B.Cu") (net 9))
 (segment (start 57.5 78.7) (end 57.5 96.2) (width 0.2) (layer "B.Cu") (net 2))
 (segment (start 42 115) (end 42.5 115) (width 0.2) (layer "B.Cu") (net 2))
 (segment (start 57.5 61.2) (end 52.8 56.5) (width 0.2) (layer "B.Cu") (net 2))
 (segment (start 57.5 61.2) (end 57.5 78.7) (width 0.2) (layer "B.Cu") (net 2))
 (segment (start 40.5 56.5) (end 40.5 113.5) (width 0.2) (layer "B.Cu") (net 2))
 (segment (start 52.8 56.5) (end 40.5 56.5) (width 0.2) (layer "B.Cu") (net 2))
 (segment (start 40.5 113.5) (end 42 115) (width 0.2) (layer "B.Cu") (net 2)))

